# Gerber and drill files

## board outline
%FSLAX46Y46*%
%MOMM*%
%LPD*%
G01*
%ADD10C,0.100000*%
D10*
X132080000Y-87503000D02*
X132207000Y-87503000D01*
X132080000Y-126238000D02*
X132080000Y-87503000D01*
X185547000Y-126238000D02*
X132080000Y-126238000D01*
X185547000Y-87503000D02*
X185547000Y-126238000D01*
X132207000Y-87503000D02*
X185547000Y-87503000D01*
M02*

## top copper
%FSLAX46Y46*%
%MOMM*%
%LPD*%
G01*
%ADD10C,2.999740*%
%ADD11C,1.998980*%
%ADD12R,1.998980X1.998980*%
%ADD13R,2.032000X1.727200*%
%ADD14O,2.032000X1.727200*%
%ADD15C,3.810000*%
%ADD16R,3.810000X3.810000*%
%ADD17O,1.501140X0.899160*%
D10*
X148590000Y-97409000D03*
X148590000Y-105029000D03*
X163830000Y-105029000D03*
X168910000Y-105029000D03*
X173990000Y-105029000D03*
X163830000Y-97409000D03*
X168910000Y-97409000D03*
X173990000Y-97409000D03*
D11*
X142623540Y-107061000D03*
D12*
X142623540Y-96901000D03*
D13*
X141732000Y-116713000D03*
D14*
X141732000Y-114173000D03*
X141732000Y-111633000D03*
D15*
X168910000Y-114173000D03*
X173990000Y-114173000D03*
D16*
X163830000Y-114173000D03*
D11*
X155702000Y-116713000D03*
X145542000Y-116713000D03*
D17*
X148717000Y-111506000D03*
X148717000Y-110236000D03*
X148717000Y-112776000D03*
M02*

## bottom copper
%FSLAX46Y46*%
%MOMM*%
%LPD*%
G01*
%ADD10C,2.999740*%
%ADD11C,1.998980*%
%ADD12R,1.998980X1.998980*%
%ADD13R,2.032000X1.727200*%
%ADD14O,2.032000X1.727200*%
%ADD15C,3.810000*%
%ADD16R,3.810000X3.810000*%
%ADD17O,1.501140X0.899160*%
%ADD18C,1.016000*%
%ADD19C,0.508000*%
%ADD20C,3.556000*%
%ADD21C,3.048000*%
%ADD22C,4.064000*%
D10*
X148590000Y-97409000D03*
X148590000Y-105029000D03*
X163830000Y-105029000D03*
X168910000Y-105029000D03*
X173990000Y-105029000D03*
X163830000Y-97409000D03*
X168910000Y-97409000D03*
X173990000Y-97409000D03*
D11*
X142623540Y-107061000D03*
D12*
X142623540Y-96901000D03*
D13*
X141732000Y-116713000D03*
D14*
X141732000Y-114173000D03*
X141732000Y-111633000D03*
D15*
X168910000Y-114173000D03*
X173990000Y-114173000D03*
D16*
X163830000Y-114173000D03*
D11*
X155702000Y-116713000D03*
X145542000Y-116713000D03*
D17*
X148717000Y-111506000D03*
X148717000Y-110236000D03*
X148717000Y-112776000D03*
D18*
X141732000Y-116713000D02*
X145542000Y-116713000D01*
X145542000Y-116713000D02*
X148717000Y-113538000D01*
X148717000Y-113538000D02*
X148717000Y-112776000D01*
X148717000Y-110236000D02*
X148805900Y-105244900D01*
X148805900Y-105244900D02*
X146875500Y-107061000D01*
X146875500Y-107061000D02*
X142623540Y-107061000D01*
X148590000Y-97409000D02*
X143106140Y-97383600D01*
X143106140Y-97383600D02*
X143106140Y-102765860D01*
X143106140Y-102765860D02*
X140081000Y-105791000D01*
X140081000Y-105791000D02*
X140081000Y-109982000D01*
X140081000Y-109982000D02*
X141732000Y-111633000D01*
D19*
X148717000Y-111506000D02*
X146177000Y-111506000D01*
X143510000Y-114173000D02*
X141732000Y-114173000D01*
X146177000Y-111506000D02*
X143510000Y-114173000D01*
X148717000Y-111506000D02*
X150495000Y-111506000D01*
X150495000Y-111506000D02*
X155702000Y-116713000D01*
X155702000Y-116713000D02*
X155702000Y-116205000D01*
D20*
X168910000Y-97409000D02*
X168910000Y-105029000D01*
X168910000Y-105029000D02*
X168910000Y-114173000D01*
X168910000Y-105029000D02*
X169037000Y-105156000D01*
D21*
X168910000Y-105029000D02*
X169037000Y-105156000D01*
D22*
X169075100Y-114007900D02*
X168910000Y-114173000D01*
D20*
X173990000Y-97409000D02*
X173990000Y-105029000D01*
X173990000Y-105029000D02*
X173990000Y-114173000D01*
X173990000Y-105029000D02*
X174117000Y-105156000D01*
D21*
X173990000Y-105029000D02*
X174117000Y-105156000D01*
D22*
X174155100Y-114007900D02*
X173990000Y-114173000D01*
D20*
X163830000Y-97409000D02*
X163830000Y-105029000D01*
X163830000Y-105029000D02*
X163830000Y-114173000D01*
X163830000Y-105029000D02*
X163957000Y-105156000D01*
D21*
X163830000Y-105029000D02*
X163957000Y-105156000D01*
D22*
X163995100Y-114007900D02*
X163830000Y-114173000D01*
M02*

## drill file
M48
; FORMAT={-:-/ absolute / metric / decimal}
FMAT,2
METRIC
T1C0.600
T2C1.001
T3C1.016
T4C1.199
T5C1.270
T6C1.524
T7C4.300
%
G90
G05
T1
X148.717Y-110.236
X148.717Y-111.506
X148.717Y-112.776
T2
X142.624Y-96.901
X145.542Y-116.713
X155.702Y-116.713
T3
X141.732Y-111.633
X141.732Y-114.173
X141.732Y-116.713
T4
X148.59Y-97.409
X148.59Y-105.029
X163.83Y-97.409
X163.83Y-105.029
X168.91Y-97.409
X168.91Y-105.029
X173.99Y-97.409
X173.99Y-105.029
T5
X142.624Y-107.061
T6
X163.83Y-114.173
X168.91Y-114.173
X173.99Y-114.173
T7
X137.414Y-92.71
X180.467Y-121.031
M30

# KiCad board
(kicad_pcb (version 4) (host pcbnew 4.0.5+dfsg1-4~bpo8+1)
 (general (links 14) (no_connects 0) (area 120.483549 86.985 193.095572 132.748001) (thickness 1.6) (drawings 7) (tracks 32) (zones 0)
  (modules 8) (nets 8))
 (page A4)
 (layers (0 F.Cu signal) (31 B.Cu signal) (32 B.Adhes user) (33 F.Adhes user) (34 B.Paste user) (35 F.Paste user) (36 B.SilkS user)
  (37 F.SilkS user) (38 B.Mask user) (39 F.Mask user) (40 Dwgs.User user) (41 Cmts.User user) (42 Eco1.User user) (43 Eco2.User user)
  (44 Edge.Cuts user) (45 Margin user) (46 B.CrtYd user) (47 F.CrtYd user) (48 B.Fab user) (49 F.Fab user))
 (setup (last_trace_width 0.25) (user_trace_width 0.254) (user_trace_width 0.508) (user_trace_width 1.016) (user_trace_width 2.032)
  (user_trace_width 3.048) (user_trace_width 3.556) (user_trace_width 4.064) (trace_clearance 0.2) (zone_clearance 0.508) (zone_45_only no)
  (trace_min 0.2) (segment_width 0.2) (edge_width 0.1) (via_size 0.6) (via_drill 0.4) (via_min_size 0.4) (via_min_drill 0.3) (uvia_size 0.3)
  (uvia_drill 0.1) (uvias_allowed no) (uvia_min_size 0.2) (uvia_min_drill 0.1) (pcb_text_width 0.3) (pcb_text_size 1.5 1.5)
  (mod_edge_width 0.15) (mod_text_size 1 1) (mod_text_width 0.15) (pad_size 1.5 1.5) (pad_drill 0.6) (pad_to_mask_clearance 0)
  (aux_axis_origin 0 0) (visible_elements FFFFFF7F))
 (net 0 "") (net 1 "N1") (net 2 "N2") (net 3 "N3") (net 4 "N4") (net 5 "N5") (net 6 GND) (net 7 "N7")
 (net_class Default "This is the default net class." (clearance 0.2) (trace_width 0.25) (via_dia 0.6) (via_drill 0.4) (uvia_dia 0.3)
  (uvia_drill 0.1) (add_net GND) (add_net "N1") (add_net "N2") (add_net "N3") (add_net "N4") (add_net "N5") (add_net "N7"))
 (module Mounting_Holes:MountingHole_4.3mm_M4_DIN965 (layer F.Cu) (at 137.414 92.71)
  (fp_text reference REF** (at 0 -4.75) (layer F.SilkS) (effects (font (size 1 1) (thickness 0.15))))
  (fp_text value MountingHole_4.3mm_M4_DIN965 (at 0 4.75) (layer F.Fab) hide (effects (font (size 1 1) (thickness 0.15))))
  (pad 1 np_thru_hole circle (at 0 0) (size 4.3 4.3) (drill 4.3) (layers *.Cu *.Mask)))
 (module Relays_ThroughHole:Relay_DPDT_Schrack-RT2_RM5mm (layer F.Cu) (at 148.59 105.029)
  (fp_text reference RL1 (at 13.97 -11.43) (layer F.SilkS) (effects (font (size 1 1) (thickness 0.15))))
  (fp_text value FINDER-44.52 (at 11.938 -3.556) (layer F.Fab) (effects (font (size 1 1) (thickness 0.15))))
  (pad A1 thru_hole circle (at 0 -7.62) (size 2.99974 2.99974) (drill 1.19888) (layers *.Cu *.Mask) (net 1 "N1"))
  (pad A2 thru_hole circle (at 0 0) (size 2.99974 2.99974) (drill 1.19888) (layers *.Cu *.Mask) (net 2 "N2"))
  (pad 22 thru_hole circle (at 15.24 0) (size 2.99974 2.99974) (drill 1.19888) (layers *.Cu *.Mask) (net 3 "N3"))
  (pad 21 thru_hole circle (at 20.32 0) (size 2.99974 2.99974) (drill 1.19888) (layers *.Cu *.Mask) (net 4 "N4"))
  (pad 24 thru_hole circle (at 25.4 0) (size 2.99974 2.99974) (drill 1.19888) (layers *.Cu *.Mask) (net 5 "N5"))
  (pad 12 thru_hole circle (at 15.24 -7.62) (size 2.99974 2.99974) (drill 1.19888) (layers *.Cu *.Mask) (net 3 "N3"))
  (pad 11 thru_hole circle (at 20.32 -7.62) (size 2.99974 2.99974) (drill 1.19888) (layers *.Cu *.Mask) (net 4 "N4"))
  (pad 14 thru_hole circle (at 25.4 -7.62) (size 2.99974 2.99974) (drill 1.19888) (layers *.Cu *.Mask) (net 5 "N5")))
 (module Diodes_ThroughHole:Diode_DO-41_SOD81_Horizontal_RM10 (layer F.Cu) (at 142.621 96.901 270)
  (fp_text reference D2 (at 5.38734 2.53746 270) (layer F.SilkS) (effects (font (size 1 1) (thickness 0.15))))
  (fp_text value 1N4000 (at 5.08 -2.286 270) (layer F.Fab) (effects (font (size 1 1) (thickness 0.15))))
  (pad 2 thru_hole circle (at 10.16 -0.00254 90) (size 1.99898 1.99898) (drill 1.27) (layers *.Cu *.Mask) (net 2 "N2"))
  (pad 1 thru_hole rect (at 0 -0.00254 90) (size 1.99898 1.99898) (drill 1.00076) (layers *.Cu *.Mask) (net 1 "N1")))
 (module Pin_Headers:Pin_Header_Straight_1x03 (layer F.Cu) (at 141.732 116.713 180)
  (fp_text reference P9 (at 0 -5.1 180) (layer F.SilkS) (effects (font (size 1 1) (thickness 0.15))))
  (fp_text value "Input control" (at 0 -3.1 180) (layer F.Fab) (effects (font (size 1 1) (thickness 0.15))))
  (pad 1 thru_hole rect (at 0 0 180) (size 2.032 1.7272) (drill 1.016) (layers *.Cu *.Mask) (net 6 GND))
  (pad 2 thru_hole oval (at 0 2.54 180) (size 2.032 1.7272) (drill 1.016) (layers *.Cu *.Mask) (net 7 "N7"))
  (pad 3 thru_hole oval (at 0 5.08 180) (size 2.032 1.7272) (drill 1.016) (layers *.Cu *.Mask) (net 1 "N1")))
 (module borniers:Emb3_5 (layer F.Cu) (at 168.91 114.173)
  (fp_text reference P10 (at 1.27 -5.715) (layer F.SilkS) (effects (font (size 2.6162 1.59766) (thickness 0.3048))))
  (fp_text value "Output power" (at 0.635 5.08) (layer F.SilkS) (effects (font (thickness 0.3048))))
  (pad 2 thru_hole circle (at 0 0) (size 3.81 3.81) (drill 1.524) (layers *.Cu *.Mask F.SilkS) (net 4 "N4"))
  (pad 3 thru_hole circle (at 5.08 0) (size 3.81 3.81) (drill 1.524) (layers *.Cu *.Mask F.SilkS) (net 5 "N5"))
  (pad 1 thru_hole rect (at -5.08 0) (size 3.81 3.81) (drill 1.524) (layers *.Cu *.Mask F.SilkS) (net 3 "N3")))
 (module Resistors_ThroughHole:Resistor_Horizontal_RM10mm (layer F.Cu) (at 155.702 116.713 180)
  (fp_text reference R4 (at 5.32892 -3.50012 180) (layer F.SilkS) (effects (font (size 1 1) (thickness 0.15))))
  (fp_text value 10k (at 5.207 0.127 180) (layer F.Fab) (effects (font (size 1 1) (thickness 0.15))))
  (pad 1 thru_hole circle (at 0 0 180) (size 1.99898 1.99898) (drill 1.00076) (layers *.Cu *.SilkS *.Mask) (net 7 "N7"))
  (pad 2 thru_hole circle (at 10.16 0 180) (size 1.99898 1.99898) (drill 1.00076) (layers *.Cu *.SilkS *.Mask) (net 6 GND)))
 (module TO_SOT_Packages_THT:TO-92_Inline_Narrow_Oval (layer F.Cu) (at 148.717 112.776 90)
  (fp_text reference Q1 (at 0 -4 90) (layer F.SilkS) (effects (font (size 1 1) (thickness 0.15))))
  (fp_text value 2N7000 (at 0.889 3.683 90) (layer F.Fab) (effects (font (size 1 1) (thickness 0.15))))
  (pad 2 thru_hole oval (at 1.27 0 270) (size 0.89916 1.50114) (drill 0.6) (layers *.Cu *.Mask) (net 7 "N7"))
  (pad 3 thru_hole oval (at 2.54 0 270) (size 0.89916 1.50114) (drill 0.6) (layers *.Cu *.Mask) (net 2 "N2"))
  (pad 1 thru_hole oval (at 0 0 270) (size 0.89916 1.50114) (drill 0.6) (layers *.Cu *.Mask) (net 6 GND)))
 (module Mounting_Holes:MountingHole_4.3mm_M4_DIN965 (layer F.Cu) (at 180.467 121.031)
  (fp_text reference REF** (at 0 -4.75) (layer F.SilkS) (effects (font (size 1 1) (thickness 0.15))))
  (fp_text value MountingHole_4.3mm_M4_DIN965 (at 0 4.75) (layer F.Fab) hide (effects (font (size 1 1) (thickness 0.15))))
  (pad 1 np_thru_hole circle (at 0 0) (size 4.3 4.3) (drill 4.3) (layers *.Cu *.Mask)))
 (gr_line (start 132.08 87.503) (end 132.207 87.503) (angle 90) (layer Edge.Cuts) (width 0.1))
 (gr_line (start 132.08 126.238) (end 132.08 87.503) (angle 90) (layer Edge.Cuts) (width 0.1))
 (gr_line (start 185.547 126.238) (end 132.08 126.238) (angle 90) (layer Edge.Cuts) (width 0.1))
 (gr_line (start 185.547 87.503) (end 185.547 126.238) (angle 90) (layer Edge.Cuts) (width 0.1))
 (gr_line (start 132.207 87.503) (end 185.547 87.503) (angle 90) (layer Edge.Cuts) (width 0.1))
 (segment (start 141.732 116.713) (end 145.542 116.713) (width 1.016) (layer B.Cu) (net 6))
 (segment (start 145.542 116.713) (end 148.717 113.538) (width 1.016) (layer B.Cu) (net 6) (status 20))
 (segment (start 148.717 113.538) (end 148.717 112.776) (width 1.016) (layer B.Cu) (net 6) (status 30))
 (segment (start 148.717 110.236) (end 148.8059 105.2449) (width 1.016) (layer B.Cu) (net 2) (status 20))
 (segment (start 148.8059 105.2449) (end 146.8755 107.061) (width 1.016) (layer B.Cu) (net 2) (status 10))
 (segment (start 146.8755 107.061) (end 142.62354 107.061) (width 1.016) (layer B.Cu) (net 2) (status 20))
 (segment (start 148.59 97.409) (end 143.10614 97.3836) (width 1.016) (layer B.Cu) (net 1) (status 20))
 (segment (start 143.10614 97.3836) (end 143.10614 102.76586) (width 1.016) (layer B.Cu) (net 1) (status 10))
 (segment (start 143.10614 102.76586) (end 140.081 105.791) (width 1.016) (layer B.Cu) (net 1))
 (segment (start 140.081 105.791) (end 140.081 109.982) (width 1.016) (layer B.Cu) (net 1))
 (segment (start 140.081 109.982) (end 141.732 111.633) (width 1.016) (layer B.Cu) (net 1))
 (segment (start 148.717 111.506) (end 146.177 111.506) (width 0.508) (layer B.Cu) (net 7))
 (segment (start 143.51 114.173) (end 141.732 114.173) (width 0.508) (layer B.Cu) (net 7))
 (segment (start 146.177 111.506) (end 143.51 114.173) (width 0.508) (layer B.Cu) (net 7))
 (segment (start 148.717 111.506) (end 150.495 111.506) (width 0.508) (layer B.Cu) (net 7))
 (segment (start 150.495 111.506) (end 155.702 116.713) (width 0.508) (layer B.Cu) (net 7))
 (segment (start 155.702 116.713) (end 155.702 116.205) (width 0.508) (layer B.Cu) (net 7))
 (segment (start 168.91 97.409) (end 168.91 105.029) (width 3.556) (layer B.Cu) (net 4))
 (segment (start 168.91 105.029) (end 168.91 114.173) (width 3.556) (layer B.Cu) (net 4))
 (segment (start 168.91 105.029) (end 169.037 105.156) (width 3.556) (layer B.Cu) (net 4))
 (segment (start 168.91 105.029) (end 169.037 105.156) (width 3.048) (layer B.Cu) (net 4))
 (segment (start 169.0751 114.0079) (end 168.91 114.173) (width 4.064) (layer B.Cu) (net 4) (status 30))
 (segment (start 173.99 97.409) (end 173.99 105.029) (width 3.556) (layer B.Cu) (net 5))
 (segment (start 173.99 105.029) (end 173.99 114.173) (width 3.556) (layer B.Cu) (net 5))
 (segment (start 173.99 105.029) (end 174.117 105.156) (width 3.556) (layer B.Cu) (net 5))
 (segment (start 173.99 105.029) (end 174.117 105.156) (width 3.048) (layer B.Cu) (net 5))
 (segment (start 174.1551 114.0079) (end 173.99 114.173) (width 4.064) (layer B.Cu) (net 5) (status 30))
 (segment (start 163.83 97.409) (end 163.83 105.029) (width 3.556) (layer B.Cu) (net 3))
 (segment (start 163.83 105.029) (end 163.83 114.173) (width 3.556) (layer B.Cu) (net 3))
 (segment (start 163.83 105.029) (end 163.957 105.156) (width 3.556) (layer B.Cu) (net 3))
 (segment (start 163.83 105.029) (end 163.957 105.156) (width 3.048) (layer B.Cu) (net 3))
 (segment (start 163.9951 114.0079) (end 163.83 114.173) (width 4.064) (layer B.Cu) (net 3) (status 30)))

